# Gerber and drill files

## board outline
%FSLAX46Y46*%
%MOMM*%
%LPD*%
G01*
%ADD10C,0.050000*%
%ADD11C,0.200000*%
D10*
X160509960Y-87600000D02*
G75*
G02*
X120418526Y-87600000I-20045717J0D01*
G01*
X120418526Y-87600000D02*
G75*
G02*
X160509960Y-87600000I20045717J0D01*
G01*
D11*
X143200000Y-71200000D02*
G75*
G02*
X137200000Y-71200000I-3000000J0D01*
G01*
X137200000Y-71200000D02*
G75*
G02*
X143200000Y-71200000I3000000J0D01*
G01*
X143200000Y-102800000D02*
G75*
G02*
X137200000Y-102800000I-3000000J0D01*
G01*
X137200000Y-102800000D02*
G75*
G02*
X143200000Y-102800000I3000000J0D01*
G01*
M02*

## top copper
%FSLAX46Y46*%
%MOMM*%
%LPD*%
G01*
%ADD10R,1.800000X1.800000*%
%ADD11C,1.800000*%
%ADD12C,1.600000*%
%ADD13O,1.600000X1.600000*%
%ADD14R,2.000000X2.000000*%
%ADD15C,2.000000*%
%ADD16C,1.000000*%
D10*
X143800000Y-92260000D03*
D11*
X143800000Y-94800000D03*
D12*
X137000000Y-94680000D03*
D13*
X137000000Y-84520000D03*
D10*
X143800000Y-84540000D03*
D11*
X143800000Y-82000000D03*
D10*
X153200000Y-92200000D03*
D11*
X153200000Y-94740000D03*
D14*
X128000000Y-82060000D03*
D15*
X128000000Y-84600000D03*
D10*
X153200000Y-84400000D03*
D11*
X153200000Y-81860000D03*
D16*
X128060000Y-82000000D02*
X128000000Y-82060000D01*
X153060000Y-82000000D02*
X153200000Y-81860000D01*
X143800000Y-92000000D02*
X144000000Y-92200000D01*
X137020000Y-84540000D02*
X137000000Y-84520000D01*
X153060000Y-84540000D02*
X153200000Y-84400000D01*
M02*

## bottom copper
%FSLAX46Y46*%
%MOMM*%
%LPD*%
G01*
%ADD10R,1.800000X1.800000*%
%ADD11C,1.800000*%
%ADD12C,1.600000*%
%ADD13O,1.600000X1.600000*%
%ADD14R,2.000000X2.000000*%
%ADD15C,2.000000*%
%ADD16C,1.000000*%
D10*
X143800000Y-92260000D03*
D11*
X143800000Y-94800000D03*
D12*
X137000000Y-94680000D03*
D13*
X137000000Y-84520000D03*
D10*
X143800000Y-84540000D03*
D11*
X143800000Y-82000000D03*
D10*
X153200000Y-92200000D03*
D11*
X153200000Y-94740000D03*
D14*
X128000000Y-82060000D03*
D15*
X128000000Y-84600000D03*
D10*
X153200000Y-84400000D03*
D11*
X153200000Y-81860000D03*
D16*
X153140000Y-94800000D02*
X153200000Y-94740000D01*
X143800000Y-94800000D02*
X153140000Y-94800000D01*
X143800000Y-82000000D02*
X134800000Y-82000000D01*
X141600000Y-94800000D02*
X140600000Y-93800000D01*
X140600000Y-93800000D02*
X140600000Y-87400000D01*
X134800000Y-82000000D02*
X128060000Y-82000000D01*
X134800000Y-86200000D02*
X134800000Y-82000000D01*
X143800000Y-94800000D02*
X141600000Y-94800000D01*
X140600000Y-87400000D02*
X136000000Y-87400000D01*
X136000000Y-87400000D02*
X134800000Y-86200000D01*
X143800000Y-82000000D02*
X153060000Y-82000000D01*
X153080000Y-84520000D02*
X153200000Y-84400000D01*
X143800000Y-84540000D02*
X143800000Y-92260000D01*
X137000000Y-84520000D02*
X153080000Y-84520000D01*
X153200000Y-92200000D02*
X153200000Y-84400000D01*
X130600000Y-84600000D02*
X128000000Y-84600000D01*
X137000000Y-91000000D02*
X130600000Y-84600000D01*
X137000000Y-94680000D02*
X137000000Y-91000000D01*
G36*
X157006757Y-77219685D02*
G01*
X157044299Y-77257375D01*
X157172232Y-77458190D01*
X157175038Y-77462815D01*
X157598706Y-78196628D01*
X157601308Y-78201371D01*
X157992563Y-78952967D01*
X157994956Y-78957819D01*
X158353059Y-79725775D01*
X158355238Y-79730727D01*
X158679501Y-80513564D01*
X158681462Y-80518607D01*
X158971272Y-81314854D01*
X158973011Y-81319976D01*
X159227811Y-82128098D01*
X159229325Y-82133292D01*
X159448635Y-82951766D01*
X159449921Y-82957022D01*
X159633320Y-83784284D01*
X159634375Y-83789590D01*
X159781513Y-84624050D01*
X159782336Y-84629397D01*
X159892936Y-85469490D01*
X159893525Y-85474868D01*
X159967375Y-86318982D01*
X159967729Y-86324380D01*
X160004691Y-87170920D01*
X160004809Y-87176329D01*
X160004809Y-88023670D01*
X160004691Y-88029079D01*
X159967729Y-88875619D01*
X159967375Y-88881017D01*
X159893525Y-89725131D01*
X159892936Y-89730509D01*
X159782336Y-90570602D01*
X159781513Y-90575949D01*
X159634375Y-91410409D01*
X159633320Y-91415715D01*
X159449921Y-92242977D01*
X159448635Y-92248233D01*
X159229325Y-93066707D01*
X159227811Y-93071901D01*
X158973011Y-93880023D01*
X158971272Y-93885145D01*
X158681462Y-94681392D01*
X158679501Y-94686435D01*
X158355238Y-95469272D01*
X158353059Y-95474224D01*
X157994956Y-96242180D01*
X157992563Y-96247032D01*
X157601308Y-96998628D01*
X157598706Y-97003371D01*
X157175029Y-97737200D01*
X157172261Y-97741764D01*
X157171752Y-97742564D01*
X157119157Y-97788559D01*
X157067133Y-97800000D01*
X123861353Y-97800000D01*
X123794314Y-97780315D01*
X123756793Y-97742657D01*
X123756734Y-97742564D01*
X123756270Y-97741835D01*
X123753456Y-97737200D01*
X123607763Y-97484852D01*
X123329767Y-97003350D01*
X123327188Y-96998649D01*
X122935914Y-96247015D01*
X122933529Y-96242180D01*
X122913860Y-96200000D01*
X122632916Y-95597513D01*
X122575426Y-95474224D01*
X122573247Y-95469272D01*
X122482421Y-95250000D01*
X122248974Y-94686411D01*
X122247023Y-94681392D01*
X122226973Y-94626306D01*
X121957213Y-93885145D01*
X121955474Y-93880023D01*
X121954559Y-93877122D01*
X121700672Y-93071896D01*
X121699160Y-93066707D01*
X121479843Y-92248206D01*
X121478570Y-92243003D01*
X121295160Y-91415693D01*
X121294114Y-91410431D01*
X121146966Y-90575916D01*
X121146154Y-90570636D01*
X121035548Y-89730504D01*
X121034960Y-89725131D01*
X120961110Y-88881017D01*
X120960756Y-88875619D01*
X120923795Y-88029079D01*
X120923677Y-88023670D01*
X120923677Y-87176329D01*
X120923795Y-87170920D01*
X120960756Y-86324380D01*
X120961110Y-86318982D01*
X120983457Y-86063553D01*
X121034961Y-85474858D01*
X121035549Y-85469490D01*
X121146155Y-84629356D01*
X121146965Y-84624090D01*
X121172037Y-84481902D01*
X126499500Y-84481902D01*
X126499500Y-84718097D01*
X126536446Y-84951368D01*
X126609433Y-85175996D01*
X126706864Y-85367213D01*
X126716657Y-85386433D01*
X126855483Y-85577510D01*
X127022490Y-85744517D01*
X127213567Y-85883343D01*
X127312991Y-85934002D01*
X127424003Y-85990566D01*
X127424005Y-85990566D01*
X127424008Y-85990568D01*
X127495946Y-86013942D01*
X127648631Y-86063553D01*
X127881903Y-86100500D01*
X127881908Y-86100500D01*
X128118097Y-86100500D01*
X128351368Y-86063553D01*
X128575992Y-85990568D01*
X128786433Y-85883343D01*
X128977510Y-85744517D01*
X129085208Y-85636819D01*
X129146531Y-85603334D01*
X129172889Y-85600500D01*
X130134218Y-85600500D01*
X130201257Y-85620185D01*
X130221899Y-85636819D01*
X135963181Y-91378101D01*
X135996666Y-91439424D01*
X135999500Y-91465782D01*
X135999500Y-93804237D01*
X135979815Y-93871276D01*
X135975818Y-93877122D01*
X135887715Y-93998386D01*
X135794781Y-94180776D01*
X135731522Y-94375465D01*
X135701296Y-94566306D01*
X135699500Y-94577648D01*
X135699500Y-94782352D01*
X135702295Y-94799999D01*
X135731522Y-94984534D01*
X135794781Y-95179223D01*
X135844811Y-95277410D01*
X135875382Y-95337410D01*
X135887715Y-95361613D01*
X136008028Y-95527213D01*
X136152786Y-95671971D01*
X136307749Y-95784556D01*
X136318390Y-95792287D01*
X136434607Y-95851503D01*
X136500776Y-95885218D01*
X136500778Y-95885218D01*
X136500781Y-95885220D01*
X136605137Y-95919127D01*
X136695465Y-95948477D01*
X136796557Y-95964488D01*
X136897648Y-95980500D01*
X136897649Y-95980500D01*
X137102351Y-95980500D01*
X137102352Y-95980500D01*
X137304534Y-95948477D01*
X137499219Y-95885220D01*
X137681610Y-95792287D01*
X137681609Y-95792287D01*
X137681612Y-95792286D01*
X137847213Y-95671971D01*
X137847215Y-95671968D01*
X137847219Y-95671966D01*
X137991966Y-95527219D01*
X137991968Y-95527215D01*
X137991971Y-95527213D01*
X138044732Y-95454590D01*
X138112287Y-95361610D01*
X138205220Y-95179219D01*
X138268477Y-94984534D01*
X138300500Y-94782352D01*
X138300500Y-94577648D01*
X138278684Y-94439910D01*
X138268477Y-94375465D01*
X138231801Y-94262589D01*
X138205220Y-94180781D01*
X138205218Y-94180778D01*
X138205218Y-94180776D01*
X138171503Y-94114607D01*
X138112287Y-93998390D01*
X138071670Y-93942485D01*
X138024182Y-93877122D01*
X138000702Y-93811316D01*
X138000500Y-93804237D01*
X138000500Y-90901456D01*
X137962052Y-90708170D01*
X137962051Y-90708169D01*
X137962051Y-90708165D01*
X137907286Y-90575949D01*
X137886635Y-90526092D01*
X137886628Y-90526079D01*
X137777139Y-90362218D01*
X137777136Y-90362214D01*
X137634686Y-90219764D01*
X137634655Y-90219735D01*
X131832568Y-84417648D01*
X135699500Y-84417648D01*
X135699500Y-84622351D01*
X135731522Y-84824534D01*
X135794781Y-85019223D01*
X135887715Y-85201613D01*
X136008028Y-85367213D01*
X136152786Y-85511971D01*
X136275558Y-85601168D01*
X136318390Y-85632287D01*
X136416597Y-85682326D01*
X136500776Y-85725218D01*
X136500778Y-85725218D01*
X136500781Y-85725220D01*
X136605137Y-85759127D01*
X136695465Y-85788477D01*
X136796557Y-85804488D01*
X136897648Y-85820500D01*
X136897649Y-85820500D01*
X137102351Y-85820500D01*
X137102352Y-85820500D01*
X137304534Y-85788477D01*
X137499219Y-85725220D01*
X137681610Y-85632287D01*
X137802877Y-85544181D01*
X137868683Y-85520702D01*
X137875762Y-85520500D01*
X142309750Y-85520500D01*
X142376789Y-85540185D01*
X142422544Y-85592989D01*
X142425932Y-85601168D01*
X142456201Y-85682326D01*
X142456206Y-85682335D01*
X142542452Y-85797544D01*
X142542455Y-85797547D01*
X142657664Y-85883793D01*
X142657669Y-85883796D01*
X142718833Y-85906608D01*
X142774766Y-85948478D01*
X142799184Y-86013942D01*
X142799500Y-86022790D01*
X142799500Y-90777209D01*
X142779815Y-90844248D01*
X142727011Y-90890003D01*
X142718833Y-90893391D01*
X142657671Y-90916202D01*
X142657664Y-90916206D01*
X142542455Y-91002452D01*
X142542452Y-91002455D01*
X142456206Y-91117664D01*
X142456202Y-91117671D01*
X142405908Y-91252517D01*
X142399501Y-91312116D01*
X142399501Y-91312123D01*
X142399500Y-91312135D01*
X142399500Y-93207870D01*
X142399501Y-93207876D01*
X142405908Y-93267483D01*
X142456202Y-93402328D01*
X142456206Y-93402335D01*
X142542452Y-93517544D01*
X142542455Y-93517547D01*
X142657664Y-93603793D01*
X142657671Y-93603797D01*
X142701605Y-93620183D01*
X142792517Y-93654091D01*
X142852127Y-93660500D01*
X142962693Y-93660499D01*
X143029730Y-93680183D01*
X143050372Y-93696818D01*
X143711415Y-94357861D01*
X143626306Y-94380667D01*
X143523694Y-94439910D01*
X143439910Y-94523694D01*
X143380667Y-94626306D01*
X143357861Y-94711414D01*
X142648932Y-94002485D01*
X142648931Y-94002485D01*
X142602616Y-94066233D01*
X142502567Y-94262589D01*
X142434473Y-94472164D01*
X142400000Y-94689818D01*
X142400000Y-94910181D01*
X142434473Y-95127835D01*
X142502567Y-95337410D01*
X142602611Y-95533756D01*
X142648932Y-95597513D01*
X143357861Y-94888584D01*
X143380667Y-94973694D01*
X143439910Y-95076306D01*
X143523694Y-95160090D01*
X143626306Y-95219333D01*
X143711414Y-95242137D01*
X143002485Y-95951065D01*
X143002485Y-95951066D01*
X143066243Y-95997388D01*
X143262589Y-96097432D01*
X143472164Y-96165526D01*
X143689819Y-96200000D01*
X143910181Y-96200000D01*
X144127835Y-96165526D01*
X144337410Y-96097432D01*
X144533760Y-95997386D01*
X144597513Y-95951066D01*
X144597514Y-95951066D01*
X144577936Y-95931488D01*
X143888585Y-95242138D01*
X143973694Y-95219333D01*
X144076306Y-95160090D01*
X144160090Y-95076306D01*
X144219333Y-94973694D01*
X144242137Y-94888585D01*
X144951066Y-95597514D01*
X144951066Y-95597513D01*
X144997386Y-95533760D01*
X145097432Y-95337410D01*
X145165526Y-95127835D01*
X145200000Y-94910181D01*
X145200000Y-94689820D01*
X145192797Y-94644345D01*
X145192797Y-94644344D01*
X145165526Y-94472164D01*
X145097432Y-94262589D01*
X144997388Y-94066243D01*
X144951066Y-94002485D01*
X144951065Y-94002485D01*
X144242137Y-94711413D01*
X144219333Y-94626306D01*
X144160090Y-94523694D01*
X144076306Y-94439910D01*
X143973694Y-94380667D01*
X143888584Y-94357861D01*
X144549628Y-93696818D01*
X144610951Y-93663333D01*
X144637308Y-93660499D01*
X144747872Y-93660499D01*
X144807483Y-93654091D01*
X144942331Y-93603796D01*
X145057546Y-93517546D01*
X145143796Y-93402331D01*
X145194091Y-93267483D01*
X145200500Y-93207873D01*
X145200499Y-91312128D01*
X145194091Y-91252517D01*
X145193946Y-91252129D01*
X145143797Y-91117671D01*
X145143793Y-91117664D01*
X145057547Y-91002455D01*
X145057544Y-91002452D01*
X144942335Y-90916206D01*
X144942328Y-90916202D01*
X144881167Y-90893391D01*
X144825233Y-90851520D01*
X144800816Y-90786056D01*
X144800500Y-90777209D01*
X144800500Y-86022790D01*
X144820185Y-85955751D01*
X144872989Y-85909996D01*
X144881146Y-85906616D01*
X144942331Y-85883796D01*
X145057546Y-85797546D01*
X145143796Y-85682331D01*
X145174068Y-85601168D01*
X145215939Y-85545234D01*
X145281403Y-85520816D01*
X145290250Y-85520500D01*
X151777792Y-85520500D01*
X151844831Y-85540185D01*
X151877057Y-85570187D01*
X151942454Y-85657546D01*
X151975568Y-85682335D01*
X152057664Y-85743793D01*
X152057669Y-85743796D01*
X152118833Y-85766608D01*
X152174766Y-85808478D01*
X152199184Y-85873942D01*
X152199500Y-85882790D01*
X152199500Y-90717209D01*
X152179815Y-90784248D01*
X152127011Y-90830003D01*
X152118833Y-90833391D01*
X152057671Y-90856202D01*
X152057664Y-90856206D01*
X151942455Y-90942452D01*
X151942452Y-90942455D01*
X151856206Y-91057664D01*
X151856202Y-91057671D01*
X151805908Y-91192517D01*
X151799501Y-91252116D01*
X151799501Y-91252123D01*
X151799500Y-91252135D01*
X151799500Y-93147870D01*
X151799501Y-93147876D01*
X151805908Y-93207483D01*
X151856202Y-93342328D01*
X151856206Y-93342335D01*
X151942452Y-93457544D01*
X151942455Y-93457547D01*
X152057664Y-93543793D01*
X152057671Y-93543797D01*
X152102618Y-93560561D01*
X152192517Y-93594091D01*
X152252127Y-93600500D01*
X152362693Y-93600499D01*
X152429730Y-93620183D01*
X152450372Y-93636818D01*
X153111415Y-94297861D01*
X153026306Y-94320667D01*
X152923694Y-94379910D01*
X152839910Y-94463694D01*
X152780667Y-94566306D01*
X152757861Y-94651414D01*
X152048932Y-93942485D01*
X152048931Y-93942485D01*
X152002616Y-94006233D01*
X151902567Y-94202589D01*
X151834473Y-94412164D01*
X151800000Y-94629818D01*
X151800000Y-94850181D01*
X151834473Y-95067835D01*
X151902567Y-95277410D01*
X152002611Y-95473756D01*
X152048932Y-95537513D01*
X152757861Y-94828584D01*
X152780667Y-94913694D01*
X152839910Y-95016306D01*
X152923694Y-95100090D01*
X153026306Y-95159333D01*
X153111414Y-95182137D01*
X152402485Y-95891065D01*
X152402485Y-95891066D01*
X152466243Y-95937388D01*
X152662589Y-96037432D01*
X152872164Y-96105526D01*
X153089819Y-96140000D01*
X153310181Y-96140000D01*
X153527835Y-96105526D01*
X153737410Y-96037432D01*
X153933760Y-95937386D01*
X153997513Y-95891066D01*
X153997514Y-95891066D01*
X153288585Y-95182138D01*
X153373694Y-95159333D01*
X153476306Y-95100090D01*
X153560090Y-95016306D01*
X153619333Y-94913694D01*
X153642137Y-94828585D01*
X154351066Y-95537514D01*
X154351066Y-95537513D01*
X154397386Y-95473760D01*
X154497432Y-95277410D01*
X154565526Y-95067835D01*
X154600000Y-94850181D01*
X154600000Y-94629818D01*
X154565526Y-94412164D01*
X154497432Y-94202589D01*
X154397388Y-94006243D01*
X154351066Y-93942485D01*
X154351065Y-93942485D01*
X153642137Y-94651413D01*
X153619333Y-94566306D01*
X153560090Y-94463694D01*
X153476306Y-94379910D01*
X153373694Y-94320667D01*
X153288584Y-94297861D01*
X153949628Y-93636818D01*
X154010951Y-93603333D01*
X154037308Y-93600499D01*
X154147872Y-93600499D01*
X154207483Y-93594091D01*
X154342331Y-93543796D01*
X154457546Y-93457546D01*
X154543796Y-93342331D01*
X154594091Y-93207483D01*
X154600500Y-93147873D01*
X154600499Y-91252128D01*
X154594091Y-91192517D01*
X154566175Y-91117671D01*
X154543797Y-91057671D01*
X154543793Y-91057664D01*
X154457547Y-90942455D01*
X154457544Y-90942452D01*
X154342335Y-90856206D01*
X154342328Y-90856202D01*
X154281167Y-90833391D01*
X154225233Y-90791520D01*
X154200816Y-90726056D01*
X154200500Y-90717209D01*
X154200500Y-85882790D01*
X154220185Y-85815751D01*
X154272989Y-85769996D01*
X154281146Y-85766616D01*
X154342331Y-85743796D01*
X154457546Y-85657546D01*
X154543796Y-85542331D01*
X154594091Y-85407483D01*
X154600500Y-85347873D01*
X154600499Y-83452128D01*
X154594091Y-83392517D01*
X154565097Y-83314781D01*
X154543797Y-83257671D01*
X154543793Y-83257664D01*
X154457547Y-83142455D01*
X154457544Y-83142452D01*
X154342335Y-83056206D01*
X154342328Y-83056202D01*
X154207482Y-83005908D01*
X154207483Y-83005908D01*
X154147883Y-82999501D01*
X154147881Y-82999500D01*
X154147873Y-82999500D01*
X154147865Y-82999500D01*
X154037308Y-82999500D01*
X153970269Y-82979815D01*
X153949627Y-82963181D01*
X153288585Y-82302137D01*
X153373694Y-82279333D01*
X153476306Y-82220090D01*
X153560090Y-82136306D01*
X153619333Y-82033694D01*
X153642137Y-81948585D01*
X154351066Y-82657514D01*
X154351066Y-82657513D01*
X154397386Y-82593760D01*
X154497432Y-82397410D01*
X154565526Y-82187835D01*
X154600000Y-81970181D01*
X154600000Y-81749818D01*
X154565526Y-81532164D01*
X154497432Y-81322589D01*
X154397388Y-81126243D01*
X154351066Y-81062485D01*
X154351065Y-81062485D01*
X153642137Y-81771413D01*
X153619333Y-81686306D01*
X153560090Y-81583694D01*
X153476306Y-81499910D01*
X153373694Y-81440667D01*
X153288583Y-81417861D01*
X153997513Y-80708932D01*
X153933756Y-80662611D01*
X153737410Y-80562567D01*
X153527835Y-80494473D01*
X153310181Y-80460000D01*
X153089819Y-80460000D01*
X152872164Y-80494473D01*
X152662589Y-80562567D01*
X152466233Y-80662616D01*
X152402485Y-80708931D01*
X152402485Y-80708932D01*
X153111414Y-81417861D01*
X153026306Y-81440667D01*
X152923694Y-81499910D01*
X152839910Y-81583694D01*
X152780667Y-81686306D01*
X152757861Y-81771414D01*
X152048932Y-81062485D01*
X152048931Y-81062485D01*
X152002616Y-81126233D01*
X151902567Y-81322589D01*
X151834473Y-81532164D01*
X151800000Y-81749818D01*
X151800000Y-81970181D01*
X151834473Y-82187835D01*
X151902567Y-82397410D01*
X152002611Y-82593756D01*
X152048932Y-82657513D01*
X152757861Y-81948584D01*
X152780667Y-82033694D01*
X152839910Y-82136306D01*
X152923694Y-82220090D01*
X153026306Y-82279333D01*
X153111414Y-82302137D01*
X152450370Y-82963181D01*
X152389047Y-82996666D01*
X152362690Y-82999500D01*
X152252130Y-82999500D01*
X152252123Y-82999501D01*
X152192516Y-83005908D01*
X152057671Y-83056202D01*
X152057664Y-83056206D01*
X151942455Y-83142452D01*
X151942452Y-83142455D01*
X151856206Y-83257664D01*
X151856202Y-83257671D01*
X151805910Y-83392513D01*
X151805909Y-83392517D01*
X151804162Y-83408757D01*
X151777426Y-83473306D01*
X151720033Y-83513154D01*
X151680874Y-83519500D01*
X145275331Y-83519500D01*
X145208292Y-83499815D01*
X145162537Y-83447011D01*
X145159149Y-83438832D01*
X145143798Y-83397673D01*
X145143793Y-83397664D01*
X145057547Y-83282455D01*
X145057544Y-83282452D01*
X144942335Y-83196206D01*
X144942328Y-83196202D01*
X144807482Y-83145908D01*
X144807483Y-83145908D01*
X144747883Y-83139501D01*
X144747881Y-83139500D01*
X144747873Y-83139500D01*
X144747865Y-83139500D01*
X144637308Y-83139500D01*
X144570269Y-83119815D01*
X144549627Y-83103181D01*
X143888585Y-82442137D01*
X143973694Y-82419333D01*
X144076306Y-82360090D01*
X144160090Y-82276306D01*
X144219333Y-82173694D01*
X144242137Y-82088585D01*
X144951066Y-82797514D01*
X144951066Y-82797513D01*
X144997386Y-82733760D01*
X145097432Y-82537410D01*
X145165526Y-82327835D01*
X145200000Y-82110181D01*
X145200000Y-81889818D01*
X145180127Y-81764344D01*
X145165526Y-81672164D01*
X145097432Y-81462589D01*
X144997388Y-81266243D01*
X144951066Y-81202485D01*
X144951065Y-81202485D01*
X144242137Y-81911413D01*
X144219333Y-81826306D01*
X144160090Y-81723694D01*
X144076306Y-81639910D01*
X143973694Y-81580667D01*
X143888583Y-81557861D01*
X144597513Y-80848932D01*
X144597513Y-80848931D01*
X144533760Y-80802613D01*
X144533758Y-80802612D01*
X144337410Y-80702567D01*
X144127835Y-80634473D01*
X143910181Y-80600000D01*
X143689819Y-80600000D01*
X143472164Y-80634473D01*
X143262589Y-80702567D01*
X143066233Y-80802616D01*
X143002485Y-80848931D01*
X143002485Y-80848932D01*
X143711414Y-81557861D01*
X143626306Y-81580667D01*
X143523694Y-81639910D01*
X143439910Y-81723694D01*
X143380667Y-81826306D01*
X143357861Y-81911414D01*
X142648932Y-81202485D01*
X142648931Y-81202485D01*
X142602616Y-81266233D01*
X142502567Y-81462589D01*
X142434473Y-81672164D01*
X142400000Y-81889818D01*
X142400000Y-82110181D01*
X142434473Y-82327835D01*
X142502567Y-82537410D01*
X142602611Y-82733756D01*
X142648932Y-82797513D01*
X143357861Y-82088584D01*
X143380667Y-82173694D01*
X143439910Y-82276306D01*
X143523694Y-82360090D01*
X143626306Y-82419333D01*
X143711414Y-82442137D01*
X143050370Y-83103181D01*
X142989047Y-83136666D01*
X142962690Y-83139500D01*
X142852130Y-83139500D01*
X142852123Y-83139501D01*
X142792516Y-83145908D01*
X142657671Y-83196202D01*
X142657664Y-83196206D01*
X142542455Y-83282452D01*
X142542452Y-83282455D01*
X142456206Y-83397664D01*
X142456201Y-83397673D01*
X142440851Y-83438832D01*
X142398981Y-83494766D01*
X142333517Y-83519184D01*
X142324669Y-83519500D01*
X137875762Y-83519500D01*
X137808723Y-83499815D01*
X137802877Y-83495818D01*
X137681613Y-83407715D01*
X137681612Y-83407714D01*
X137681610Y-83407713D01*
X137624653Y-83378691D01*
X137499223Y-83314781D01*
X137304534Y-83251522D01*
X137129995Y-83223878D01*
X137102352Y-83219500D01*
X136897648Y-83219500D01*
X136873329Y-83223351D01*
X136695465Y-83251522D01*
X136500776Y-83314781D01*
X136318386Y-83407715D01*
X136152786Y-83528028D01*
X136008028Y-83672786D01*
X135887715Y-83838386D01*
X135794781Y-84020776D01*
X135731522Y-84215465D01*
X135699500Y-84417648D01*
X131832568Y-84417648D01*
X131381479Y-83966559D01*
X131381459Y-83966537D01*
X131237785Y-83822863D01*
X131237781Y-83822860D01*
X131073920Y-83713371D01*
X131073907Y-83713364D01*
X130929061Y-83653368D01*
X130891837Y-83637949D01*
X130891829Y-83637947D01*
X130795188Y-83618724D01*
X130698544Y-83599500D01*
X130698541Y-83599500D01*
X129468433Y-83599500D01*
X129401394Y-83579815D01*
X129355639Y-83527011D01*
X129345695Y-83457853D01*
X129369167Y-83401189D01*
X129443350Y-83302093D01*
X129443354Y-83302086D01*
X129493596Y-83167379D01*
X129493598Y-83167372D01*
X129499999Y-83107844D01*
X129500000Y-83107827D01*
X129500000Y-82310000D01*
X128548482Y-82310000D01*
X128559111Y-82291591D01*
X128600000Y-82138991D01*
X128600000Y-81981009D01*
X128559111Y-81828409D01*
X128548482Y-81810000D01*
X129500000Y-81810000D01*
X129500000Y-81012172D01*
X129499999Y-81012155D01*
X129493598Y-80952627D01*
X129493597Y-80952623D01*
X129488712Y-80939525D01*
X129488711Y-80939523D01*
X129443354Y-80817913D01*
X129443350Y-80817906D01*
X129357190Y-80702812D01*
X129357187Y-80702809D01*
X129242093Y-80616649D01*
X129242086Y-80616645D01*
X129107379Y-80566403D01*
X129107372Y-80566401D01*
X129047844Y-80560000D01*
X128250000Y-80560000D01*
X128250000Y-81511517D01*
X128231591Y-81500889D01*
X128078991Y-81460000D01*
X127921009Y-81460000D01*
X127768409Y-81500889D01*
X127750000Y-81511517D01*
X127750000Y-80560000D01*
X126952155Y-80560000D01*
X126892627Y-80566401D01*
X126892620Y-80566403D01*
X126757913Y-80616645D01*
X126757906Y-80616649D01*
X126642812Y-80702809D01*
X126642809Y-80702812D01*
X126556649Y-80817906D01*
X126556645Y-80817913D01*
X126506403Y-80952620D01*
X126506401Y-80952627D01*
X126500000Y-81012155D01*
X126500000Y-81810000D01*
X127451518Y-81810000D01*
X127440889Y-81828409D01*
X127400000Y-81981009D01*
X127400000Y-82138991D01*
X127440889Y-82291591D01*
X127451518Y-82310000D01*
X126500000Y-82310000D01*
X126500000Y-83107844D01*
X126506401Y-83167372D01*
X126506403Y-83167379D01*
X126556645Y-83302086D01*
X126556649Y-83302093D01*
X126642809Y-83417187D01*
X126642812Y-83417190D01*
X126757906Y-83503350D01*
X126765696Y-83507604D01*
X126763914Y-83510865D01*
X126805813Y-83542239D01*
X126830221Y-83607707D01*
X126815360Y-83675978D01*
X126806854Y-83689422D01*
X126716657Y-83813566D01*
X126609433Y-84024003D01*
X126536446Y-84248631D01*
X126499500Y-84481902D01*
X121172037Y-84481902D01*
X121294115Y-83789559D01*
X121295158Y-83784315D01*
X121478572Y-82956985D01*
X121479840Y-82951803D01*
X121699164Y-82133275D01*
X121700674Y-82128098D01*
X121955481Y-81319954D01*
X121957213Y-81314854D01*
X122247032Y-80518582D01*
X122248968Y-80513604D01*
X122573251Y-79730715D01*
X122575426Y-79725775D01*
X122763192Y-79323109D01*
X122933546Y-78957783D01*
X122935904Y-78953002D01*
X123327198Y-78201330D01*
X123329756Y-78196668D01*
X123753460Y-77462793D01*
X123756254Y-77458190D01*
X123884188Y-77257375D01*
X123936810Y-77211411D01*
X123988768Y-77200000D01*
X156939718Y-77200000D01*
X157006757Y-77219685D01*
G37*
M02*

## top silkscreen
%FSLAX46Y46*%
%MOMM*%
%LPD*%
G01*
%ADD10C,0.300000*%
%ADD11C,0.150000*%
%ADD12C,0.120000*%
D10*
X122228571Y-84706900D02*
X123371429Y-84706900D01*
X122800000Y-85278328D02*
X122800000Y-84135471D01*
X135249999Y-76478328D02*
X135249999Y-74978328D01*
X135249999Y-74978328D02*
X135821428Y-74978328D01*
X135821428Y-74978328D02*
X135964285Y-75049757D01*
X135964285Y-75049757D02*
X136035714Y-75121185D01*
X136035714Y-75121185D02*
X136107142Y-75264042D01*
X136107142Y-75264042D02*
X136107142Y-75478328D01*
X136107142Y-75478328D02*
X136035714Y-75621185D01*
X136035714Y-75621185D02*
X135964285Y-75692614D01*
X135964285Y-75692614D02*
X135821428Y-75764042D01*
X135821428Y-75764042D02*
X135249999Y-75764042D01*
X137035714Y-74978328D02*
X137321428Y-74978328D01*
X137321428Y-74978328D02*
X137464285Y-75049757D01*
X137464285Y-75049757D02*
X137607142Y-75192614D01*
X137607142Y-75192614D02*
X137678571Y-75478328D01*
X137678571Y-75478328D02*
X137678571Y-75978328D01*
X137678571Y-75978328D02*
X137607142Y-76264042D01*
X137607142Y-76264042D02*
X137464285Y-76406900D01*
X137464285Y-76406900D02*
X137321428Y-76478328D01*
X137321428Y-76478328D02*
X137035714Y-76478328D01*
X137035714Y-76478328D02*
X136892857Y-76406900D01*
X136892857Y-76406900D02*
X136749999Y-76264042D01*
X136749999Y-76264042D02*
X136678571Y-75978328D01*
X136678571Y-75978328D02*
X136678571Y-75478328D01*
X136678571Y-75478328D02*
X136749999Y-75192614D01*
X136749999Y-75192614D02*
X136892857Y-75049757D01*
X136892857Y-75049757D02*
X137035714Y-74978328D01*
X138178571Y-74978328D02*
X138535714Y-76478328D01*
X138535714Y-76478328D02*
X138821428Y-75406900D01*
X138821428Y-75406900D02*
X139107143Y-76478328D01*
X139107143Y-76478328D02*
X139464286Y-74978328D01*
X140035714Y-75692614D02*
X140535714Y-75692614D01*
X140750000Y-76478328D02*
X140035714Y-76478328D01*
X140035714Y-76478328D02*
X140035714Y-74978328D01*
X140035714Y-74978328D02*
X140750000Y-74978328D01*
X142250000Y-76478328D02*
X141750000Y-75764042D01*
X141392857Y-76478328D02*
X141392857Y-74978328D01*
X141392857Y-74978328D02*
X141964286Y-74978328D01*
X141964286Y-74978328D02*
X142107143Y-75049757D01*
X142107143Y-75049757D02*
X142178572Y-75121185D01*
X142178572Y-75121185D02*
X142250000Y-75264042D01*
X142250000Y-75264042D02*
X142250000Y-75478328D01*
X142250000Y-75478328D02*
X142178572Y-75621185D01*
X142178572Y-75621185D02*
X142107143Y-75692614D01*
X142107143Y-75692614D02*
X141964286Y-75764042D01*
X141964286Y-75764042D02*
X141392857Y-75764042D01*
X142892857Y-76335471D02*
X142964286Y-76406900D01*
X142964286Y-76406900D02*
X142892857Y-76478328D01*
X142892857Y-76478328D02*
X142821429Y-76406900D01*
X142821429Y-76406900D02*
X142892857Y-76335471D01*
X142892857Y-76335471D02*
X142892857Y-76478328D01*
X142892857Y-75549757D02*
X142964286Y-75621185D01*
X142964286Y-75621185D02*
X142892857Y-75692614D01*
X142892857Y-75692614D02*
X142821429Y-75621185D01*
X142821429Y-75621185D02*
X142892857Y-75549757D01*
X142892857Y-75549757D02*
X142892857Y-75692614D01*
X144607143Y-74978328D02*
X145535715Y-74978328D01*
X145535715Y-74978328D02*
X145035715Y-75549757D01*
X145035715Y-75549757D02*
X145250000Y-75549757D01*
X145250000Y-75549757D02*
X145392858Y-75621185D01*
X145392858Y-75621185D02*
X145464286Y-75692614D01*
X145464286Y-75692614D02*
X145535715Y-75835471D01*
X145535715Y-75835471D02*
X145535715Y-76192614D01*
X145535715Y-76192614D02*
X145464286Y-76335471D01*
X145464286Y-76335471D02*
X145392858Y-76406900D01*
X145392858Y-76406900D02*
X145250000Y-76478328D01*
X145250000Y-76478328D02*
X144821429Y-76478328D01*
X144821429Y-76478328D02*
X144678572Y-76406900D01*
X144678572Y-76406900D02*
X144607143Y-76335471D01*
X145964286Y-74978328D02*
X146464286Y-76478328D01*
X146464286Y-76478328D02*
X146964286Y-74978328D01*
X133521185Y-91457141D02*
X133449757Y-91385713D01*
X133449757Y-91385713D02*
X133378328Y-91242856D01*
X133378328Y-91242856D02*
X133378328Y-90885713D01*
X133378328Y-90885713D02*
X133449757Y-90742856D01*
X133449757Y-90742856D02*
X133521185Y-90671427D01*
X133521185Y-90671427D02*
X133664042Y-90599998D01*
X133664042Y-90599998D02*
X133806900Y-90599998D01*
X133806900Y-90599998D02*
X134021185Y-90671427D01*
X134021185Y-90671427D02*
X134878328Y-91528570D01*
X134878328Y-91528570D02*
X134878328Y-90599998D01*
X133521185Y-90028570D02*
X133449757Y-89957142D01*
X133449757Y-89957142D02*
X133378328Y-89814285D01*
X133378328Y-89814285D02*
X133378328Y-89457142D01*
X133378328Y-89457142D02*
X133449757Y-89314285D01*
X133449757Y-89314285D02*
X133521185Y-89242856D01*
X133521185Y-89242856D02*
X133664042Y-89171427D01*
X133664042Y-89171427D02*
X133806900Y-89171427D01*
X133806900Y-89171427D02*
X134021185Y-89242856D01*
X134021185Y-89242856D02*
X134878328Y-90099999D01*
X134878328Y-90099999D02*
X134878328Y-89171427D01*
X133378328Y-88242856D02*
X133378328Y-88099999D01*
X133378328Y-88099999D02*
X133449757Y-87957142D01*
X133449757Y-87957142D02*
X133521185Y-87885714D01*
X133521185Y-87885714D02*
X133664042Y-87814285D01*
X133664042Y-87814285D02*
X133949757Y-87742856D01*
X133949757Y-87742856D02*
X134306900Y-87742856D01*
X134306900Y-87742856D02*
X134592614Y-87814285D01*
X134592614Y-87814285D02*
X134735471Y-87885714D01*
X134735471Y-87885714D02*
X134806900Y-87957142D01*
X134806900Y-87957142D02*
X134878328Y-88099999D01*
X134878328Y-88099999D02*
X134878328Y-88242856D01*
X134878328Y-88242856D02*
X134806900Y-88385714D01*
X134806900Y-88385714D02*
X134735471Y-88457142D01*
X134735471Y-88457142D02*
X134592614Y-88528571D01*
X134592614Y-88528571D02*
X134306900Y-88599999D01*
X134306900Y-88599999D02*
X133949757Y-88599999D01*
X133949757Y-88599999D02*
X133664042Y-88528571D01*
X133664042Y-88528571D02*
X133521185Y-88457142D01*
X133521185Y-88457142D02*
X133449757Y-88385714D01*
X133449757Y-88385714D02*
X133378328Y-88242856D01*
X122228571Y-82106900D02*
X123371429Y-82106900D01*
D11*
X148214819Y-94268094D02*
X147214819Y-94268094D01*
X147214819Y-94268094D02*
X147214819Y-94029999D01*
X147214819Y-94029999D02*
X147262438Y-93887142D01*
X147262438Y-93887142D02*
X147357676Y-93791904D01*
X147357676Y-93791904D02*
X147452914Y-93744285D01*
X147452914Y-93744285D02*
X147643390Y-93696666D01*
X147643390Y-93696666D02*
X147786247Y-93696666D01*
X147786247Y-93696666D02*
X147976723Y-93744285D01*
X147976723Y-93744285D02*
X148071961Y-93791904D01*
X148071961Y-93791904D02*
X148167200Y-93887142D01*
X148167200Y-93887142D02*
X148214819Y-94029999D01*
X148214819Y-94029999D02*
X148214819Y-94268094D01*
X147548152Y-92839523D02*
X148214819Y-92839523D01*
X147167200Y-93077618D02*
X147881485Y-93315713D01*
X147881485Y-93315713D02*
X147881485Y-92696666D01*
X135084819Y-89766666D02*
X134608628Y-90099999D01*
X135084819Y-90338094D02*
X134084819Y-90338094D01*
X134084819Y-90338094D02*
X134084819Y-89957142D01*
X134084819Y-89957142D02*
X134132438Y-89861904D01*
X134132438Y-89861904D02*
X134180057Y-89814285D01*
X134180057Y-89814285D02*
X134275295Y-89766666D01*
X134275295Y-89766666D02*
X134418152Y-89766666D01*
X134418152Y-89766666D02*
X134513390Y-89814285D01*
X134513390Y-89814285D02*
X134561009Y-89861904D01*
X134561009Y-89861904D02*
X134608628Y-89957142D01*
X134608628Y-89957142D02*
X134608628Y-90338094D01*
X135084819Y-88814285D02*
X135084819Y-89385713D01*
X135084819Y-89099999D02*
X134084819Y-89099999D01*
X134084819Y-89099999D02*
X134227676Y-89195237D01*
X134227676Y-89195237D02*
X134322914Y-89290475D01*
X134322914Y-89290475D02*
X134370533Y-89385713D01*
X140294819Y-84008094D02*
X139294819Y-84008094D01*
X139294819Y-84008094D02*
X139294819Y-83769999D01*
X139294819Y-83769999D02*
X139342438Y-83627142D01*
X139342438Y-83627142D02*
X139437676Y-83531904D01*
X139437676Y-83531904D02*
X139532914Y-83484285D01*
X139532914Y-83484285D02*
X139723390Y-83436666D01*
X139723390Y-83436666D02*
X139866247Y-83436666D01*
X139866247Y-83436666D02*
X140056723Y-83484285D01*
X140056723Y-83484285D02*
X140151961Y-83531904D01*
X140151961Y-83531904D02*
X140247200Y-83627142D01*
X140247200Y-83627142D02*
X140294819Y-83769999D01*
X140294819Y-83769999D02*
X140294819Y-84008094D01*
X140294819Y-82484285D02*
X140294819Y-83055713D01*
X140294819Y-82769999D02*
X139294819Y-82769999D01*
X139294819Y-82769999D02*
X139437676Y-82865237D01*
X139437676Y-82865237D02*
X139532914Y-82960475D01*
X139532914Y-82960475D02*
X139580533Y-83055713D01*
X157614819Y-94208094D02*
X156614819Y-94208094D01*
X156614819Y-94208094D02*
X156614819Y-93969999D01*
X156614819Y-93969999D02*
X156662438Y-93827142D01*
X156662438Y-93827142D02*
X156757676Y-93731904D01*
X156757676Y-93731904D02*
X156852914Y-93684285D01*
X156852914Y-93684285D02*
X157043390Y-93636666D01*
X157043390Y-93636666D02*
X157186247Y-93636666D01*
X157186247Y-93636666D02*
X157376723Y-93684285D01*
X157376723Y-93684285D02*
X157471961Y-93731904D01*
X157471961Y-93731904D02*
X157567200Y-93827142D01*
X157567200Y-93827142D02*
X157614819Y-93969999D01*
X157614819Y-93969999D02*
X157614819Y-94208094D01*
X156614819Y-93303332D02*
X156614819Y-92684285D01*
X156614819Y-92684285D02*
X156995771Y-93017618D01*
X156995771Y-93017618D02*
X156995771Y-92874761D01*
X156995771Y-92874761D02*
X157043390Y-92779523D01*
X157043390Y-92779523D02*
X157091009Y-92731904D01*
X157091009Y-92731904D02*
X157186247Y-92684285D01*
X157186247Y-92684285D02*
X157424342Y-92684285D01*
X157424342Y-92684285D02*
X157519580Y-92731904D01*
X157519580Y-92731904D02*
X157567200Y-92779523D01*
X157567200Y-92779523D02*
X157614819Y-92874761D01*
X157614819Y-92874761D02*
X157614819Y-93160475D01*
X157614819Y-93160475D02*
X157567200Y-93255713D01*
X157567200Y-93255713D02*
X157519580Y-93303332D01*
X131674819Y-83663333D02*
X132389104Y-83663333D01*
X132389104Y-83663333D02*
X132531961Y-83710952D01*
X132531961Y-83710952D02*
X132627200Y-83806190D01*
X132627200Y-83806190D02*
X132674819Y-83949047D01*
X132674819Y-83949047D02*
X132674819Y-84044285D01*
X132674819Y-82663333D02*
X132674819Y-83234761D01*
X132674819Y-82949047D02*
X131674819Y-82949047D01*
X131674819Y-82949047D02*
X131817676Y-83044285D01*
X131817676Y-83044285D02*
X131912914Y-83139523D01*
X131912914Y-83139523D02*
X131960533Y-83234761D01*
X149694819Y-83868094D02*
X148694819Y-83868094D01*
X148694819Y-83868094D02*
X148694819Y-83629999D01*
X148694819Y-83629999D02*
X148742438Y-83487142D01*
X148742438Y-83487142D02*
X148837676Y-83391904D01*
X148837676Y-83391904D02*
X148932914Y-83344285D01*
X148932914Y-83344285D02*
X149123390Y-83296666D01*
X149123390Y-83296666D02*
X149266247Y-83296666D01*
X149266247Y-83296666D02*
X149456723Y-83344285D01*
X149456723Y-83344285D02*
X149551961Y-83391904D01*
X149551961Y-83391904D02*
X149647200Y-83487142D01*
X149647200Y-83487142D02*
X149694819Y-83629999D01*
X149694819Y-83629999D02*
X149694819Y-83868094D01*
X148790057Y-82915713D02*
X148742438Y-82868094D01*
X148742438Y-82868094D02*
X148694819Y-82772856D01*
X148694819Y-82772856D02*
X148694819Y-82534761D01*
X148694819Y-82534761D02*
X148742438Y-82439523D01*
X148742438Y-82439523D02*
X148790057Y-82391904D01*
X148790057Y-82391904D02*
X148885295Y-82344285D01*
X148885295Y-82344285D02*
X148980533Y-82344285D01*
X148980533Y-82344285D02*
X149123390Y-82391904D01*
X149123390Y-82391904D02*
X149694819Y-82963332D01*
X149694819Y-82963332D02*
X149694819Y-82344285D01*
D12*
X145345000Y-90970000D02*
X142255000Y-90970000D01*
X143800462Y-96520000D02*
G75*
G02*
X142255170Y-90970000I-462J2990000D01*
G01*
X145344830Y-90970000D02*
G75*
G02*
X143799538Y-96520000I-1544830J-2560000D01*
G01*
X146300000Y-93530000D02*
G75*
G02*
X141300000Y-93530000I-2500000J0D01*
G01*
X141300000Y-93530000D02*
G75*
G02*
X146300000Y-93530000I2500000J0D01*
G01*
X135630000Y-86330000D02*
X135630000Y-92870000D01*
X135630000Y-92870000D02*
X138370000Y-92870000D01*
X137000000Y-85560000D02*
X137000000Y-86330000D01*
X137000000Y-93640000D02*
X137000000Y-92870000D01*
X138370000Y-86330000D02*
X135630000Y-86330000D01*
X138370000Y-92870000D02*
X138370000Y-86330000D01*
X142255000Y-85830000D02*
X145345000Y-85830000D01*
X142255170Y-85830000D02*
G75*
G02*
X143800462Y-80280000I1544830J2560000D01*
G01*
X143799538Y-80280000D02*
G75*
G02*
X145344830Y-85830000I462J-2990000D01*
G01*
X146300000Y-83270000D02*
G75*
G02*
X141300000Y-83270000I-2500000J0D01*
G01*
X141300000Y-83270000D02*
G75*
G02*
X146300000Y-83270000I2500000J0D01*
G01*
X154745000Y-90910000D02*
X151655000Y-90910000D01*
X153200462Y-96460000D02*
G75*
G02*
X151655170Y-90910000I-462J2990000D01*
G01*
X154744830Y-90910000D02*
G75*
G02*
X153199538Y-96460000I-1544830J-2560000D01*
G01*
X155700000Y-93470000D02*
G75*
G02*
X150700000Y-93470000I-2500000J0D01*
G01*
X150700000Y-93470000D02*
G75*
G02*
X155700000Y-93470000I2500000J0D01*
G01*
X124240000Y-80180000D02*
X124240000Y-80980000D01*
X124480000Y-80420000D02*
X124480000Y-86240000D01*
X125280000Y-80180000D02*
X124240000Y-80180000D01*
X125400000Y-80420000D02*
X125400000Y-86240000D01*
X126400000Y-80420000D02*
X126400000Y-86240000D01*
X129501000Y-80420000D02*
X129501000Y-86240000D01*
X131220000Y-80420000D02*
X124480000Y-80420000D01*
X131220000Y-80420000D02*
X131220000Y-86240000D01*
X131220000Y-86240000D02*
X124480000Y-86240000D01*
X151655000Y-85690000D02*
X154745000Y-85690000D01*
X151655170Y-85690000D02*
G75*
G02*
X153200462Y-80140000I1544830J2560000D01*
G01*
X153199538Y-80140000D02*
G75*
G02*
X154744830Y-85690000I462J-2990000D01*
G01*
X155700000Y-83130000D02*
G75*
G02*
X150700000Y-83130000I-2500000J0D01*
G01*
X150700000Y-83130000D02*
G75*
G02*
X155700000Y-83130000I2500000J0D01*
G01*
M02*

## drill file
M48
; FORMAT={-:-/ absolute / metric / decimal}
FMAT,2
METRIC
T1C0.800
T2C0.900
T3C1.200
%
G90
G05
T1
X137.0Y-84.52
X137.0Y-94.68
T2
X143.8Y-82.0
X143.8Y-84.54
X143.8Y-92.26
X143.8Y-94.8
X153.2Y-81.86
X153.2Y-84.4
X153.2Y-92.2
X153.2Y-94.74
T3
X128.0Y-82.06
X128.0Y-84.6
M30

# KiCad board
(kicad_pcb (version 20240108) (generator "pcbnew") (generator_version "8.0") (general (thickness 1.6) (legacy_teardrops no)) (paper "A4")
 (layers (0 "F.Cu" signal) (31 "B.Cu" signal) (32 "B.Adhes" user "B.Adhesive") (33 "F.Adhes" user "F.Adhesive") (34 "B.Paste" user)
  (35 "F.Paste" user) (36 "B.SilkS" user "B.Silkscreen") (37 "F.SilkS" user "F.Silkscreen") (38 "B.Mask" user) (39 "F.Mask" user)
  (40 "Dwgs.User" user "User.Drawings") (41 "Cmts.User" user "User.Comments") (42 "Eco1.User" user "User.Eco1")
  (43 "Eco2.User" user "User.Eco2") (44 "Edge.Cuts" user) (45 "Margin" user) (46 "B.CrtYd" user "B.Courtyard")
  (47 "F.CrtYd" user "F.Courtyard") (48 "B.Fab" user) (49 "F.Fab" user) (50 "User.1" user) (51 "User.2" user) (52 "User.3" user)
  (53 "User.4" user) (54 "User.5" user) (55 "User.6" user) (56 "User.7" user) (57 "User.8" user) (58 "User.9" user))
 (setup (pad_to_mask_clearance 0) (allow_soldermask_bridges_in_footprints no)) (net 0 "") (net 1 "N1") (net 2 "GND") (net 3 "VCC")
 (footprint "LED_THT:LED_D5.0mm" (layer "F.Cu") (at 143.8 92.26 -90)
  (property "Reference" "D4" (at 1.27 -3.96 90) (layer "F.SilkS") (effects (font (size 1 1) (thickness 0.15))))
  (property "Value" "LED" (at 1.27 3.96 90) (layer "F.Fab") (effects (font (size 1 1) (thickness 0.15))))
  (fp_line (start -1.29 -1.545) (end -1.29 1.545) (stroke (width 0.12) (type solid)) (layer "F.SilkS"))
  (fp_arc (start 4.26 -0.000462) (mid 2.072002 2.880433) (end -1.29 1.54483) (stroke (width 0.12) (type solid)) (layer "F.SilkS"))
  (fp_arc (start -1.29 -1.54483) (mid 2.072002 -2.880433) (end 4.26 0.000462) (stroke (width 0.12) (type solid)) (layer "F.SilkS"))
  (fp_circle (center 1.27 0) (end 3.77 0) (stroke (width 0.12) (type solid)) (fill none) (layer "F.SilkS"))
  (pad "1" thru_hole rect (at 0 0 270) (size 1.8 1.8) (drill 0.9) (layers "*.Cu" "*.Mask") (remove_unused_layers no) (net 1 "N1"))
  (pad "2" thru_hole circle (at 2.54 0 270) (size 1.8 1.8) (drill 0.9) (layers "*.Cu" "*.Mask") (remove_unused_layers no) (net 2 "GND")))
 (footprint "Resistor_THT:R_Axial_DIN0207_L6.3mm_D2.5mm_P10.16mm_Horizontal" (layer "F.Cu") (at 137 94.68 90)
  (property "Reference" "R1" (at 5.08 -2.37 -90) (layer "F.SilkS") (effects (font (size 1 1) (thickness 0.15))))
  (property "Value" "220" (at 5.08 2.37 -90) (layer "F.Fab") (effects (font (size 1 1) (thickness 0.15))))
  (fp_line (start 8.35 -1.37) (end 1.81 -1.37) (stroke (width 0.12) (type solid)) (layer "F.SilkS"))
  (fp_line (start 1.81 -1.37) (end 1.81 1.37) (stroke (width 0.12) (type solid)) (layer "F.SilkS"))
  (fp_line (start 9.12 0) (end 8.35 0) (stroke (width 0.12) (type solid)) (layer "F.SilkS"))
  (fp_line (start 1.04 0) (end 1.81 0) (stroke (width 0.12) (type solid)) (layer "F.SilkS"))
  (fp_line (start 8.35 1.37) (end 8.35 -1.37) (stroke (width 0.12) (type solid)) (layer "F.SilkS"))
  (fp_line (start 1.81 1.37) (end 8.35 1.37) (stroke (width 0.12) (type solid)) (layer "F.SilkS"))
  (pad "1" thru_hole circle (at 0 0 90) (size 1.6 1.6) (drill 0.8) (layers "*.Cu" "*.Mask") (remove_unused_layers no) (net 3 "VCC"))
  (pad "2" thru_hole oval (at 10.16 0 90) (size 1.6 1.6) (drill 0.8) (layers "*.Cu" "*.Mask") (remove_unused_layers no) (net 1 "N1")))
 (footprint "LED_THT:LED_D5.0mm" (layer "F.Cu") (at 143.8 84.54 90)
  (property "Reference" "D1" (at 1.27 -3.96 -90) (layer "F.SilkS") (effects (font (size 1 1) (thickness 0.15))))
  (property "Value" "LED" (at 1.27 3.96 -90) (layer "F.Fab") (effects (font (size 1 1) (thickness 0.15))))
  (fp_line (start -1.29 -1.545) (end -1.29 1.545) (stroke (width 0.12) (type solid)) (layer "F.SilkS"))
  (fp_arc (start -1.29 -1.54483) (mid 2.072002 -2.880433) (end 4.26 0.000462) (stroke (width 0.12) (type solid)) (layer "F.SilkS"))
  (fp_arc (start 4.26 -0.000462) (mid 2.072002 2.880433) (end -1.29 1.54483) (stroke (width 0.12) (type solid)) (layer "F.SilkS"))
  (fp_circle (center 1.27 0) (end 3.77 0) (stroke (width 0.12) (type solid)) (fill none) (layer "F.SilkS"))
  (pad "1" thru_hole rect (at 0 0 90) (size 1.8 1.8) (drill 0.9) (layers "*.Cu" "*.Mask") (remove_unused_layers no) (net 1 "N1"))
  (pad "2" thru_hole circle (at 2.54 0 90) (size 1.8 1.8) (drill 0.9) (layers "*.Cu" "*.Mask") (remove_unused_layers no) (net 2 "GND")))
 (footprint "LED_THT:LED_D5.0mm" (layer "F.Cu") (at 153.2 92.2 -90)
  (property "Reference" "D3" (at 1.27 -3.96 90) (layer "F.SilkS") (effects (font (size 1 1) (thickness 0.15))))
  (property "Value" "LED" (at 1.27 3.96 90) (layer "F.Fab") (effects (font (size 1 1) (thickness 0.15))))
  (fp_line (start -1.29 -1.545) (end -1.29 1.545) (stroke (width 0.12) (type solid)) (layer "F.SilkS"))
  (fp_arc (start 4.26 -0.000462) (mid 2.072002 2.880433) (end -1.29 1.54483) (stroke (width 0.12) (type solid)) (layer "F.SilkS"))
  (fp_arc (start -1.29 -1.54483) (mid 2.072002 -2.880433) (end 4.26 0.000462) (stroke (width 0.12) (type solid)) (layer "F.SilkS"))
  (fp_circle (center 1.27 0) (end 3.77 0) (stroke (width 0.12) (type solid)) (fill none) (layer "F.SilkS"))
  (pad "1" thru_hole rect (at 0 0 270) (size 1.8 1.8) (drill 0.9) (layers "*.Cu" "*.Mask") (remove_unused_layers no) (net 1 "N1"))
  (pad "2" thru_hole circle (at 2.54 0 270) (size 1.8 1.8) (drill 0.9) (layers "*.Cu" "*.Mask") (remove_unused_layers no) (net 2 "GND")))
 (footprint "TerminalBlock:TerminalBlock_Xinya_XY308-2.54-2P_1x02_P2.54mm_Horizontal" (layer "F.Cu") (at 128 82.06 -90)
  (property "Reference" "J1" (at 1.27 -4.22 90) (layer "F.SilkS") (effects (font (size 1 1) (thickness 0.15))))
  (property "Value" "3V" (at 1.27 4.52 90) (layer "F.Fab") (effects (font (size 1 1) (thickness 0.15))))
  (fp_line (start -1.88 3.76) (end -1.08 3.76) (stroke (width 0.12) (type solid)) (layer "F.SilkS"))
  (fp_line (start -1.64 3.52) (end 4.18 3.52) (stroke (width 0.12) (type solid)) (layer "F.SilkS"))
  (fp_line (start -1.88 2.72) (end -1.88 3.76) (stroke (width 0.12) (type solid)) (layer "F.SilkS"))
  (fp_line (start -1.64 2.6) (end 4.18 2.6) (stroke (width 0.12) (type solid)) (layer "F.SilkS"))
  (fp_line (start -1.64 1.6) (end 4.18 1.6) (stroke (width 0.12) (type solid)) (layer "F.SilkS"))
  (fp_line (start -1.64 -1.501) (end 4.18 -1.501) (stroke (width 0.12) (type solid)) (layer "F.SilkS"))
  (fp_line (start -1.64 -3.22) (end -1.64 3.52) (stroke (width 0.12) (type solid)) (layer "F.SilkS"))
  (fp_line (start -1.64 -3.22) (end 4.18 -3.22) (stroke (width 0.12) (type solid)) (layer "F.SilkS"))
  (fp_line (start 4.18 -3.22) (end 4.18 3.52) (stroke (width 0.12) (type solid)) (layer "F.SilkS"))
  (pad "1" thru_hole rect (at 0 0 270) (size 2 2) (drill 1.2) (layers "*.Cu" "*.Mask") (remove_unused_layers no) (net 2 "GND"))
  (pad "2" thru_hole circle (at 2.54 0 270) (size 2 2) (drill 1.2) (layers "*.Cu" "*.Mask") (remove_unused_layers no) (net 3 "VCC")))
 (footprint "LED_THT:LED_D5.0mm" (layer "F.Cu") (at 153.2 84.4 90)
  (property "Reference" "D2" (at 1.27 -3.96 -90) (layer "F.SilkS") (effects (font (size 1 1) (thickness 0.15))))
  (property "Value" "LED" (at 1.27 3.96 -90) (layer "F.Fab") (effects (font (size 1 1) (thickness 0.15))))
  (fp_line (start -1.29 -1.545) (end -1.29 1.545) (stroke (width 0.12) (type solid)) (layer "F.SilkS"))
  (fp_arc (start -1.29 -1.54483) (mid 2.072002 -2.880433) (end 4.26 0.000462) (stroke (width 0.12) (type solid)) (layer "F.SilkS"))
  (fp_arc (start 4.26 -0.000462) (mid 2.072002 2.880433) (end -1.29 1.54483) (stroke (width 0.12) (type solid)) (layer "F.SilkS"))
  (fp_circle (center 1.27 0) (end 3.77 0) (stroke (width 0.12) (type solid)) (fill none) (layer "F.SilkS"))
  (pad "1" thru_hole rect (at 0 0 90) (size 1.8 1.8) (drill 0.9) (layers "*.Cu" "*.Mask") (remove_unused_layers no) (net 1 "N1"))
  (pad "2" thru_hole circle (at 2.54 0 90) (size 1.8 1.8) (drill 0.9) (layers "*.Cu" "*.Mask") (remove_unused_layers no) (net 2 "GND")))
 (gr_circle (center 140.464243 87.6) (end 151.4 104.4) (stroke (width 0.05) (type default)) (fill none) (layer "Edge.Cuts"))
 (gr_circle (center 140.2 71.2) (end 143.2 71.2) (stroke (width 0.2) (type default)) (fill none) (layer "Edge.Cuts"))
 (gr_circle (center 140.2 102.8) (end 143.2 102.8) (stroke (width 0.2) (type default)) (fill none) (layer "Edge.Cuts"))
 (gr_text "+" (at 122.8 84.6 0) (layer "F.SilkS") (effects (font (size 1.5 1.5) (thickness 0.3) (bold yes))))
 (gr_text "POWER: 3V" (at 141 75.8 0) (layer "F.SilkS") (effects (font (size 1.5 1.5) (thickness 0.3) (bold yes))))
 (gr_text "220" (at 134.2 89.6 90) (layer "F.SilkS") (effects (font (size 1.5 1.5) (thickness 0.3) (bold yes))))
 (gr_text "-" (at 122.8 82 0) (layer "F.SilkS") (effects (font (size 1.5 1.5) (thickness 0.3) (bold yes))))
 (segment (start 128.06 82) (end 128 82.06) (width 1) (layer "F.Cu") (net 2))
 (segment (start 153.06 82) (end 153.2 81.86) (width 1) (layer "F.Cu") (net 2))
 (segment (start 153.14 94.8) (end 153.2 94.74) (width 1) (layer "B.Cu") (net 2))
 (segment (start 143.8 94.8) (end 153.14 94.8) (width 1) (layer "B.Cu") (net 2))
 (segment (start 143.8 82) (end 134.8 82) (width 1) (layer "B.Cu") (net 2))
 (segment (start 141.6 94.8) (end 140.6 93.8) (width 1) (layer "B.Cu") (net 2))
 (segment (start 140.6 93.8) (end 140.6 87.4) (width 1) (layer "B.Cu") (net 2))
 (segment (start 134.8 82) (end 128.06 82) (width 1) (layer "B.Cu") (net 2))
 (segment (start 134.8 86.2) (end 134.8 82) (width 1) (layer "B.Cu") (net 2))
 (segment (start 143.8 94.8) (end 141.6 94.8) (width 1) (layer "B.Cu") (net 2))
 (segment (start 140.6 87.4) (end 136 87.4) (width 1) (layer "B.Cu") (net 2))
 (segment (start 136 87.4) (end 134.8 86.2) (width 1) (layer "B.Cu") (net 2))
 (segment (start 143.8 82) (end 153.06 82) (width 1) (layer "B.Cu") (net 2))
 (segment (start 143.8 92) (end 144 92.2) (width 1) (layer "F.Cu") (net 1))
 (segment (start 137.02 84.54) (end 137 84.52) (width 1) (layer "F.Cu") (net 1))
 (segment (start 153.06 84.54) (end 153.2 84.4) (width 1) (layer "F.Cu") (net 1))
 (segment (start 153.08 84.52) (end 153.2 84.4) (width 1) (layer "B.Cu") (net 1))
 (segment (start 143.8 84.54) (end 143.8 92.26) (width 1) (layer "B.Cu") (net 1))
 (segment (start 137 84.52) (end 153.08 84.52) (width 1) (layer "B.Cu") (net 1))
 (segment (start 153.2 92.2) (end 153.2 84.4) (width 1) (layer "B.Cu") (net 1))
 (segment (start 130.6 84.6) (end 128 84.6) (width 1) (layer "B.Cu") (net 3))
 (segment (start 137 91) (end 130.6 84.6) (width 1) (layer "B.Cu") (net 3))
 (segment (start 137 94.68) (end 137 91) (width 1) (layer "B.Cu") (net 3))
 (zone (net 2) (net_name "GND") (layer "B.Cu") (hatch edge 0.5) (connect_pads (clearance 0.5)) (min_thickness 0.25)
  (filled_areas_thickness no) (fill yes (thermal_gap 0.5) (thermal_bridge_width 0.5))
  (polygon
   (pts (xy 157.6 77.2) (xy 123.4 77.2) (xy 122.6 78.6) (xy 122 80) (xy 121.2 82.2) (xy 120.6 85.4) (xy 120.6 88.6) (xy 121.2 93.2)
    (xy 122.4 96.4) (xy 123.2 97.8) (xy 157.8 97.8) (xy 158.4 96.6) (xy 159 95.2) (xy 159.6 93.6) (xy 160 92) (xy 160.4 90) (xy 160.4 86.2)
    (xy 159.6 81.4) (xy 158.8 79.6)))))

